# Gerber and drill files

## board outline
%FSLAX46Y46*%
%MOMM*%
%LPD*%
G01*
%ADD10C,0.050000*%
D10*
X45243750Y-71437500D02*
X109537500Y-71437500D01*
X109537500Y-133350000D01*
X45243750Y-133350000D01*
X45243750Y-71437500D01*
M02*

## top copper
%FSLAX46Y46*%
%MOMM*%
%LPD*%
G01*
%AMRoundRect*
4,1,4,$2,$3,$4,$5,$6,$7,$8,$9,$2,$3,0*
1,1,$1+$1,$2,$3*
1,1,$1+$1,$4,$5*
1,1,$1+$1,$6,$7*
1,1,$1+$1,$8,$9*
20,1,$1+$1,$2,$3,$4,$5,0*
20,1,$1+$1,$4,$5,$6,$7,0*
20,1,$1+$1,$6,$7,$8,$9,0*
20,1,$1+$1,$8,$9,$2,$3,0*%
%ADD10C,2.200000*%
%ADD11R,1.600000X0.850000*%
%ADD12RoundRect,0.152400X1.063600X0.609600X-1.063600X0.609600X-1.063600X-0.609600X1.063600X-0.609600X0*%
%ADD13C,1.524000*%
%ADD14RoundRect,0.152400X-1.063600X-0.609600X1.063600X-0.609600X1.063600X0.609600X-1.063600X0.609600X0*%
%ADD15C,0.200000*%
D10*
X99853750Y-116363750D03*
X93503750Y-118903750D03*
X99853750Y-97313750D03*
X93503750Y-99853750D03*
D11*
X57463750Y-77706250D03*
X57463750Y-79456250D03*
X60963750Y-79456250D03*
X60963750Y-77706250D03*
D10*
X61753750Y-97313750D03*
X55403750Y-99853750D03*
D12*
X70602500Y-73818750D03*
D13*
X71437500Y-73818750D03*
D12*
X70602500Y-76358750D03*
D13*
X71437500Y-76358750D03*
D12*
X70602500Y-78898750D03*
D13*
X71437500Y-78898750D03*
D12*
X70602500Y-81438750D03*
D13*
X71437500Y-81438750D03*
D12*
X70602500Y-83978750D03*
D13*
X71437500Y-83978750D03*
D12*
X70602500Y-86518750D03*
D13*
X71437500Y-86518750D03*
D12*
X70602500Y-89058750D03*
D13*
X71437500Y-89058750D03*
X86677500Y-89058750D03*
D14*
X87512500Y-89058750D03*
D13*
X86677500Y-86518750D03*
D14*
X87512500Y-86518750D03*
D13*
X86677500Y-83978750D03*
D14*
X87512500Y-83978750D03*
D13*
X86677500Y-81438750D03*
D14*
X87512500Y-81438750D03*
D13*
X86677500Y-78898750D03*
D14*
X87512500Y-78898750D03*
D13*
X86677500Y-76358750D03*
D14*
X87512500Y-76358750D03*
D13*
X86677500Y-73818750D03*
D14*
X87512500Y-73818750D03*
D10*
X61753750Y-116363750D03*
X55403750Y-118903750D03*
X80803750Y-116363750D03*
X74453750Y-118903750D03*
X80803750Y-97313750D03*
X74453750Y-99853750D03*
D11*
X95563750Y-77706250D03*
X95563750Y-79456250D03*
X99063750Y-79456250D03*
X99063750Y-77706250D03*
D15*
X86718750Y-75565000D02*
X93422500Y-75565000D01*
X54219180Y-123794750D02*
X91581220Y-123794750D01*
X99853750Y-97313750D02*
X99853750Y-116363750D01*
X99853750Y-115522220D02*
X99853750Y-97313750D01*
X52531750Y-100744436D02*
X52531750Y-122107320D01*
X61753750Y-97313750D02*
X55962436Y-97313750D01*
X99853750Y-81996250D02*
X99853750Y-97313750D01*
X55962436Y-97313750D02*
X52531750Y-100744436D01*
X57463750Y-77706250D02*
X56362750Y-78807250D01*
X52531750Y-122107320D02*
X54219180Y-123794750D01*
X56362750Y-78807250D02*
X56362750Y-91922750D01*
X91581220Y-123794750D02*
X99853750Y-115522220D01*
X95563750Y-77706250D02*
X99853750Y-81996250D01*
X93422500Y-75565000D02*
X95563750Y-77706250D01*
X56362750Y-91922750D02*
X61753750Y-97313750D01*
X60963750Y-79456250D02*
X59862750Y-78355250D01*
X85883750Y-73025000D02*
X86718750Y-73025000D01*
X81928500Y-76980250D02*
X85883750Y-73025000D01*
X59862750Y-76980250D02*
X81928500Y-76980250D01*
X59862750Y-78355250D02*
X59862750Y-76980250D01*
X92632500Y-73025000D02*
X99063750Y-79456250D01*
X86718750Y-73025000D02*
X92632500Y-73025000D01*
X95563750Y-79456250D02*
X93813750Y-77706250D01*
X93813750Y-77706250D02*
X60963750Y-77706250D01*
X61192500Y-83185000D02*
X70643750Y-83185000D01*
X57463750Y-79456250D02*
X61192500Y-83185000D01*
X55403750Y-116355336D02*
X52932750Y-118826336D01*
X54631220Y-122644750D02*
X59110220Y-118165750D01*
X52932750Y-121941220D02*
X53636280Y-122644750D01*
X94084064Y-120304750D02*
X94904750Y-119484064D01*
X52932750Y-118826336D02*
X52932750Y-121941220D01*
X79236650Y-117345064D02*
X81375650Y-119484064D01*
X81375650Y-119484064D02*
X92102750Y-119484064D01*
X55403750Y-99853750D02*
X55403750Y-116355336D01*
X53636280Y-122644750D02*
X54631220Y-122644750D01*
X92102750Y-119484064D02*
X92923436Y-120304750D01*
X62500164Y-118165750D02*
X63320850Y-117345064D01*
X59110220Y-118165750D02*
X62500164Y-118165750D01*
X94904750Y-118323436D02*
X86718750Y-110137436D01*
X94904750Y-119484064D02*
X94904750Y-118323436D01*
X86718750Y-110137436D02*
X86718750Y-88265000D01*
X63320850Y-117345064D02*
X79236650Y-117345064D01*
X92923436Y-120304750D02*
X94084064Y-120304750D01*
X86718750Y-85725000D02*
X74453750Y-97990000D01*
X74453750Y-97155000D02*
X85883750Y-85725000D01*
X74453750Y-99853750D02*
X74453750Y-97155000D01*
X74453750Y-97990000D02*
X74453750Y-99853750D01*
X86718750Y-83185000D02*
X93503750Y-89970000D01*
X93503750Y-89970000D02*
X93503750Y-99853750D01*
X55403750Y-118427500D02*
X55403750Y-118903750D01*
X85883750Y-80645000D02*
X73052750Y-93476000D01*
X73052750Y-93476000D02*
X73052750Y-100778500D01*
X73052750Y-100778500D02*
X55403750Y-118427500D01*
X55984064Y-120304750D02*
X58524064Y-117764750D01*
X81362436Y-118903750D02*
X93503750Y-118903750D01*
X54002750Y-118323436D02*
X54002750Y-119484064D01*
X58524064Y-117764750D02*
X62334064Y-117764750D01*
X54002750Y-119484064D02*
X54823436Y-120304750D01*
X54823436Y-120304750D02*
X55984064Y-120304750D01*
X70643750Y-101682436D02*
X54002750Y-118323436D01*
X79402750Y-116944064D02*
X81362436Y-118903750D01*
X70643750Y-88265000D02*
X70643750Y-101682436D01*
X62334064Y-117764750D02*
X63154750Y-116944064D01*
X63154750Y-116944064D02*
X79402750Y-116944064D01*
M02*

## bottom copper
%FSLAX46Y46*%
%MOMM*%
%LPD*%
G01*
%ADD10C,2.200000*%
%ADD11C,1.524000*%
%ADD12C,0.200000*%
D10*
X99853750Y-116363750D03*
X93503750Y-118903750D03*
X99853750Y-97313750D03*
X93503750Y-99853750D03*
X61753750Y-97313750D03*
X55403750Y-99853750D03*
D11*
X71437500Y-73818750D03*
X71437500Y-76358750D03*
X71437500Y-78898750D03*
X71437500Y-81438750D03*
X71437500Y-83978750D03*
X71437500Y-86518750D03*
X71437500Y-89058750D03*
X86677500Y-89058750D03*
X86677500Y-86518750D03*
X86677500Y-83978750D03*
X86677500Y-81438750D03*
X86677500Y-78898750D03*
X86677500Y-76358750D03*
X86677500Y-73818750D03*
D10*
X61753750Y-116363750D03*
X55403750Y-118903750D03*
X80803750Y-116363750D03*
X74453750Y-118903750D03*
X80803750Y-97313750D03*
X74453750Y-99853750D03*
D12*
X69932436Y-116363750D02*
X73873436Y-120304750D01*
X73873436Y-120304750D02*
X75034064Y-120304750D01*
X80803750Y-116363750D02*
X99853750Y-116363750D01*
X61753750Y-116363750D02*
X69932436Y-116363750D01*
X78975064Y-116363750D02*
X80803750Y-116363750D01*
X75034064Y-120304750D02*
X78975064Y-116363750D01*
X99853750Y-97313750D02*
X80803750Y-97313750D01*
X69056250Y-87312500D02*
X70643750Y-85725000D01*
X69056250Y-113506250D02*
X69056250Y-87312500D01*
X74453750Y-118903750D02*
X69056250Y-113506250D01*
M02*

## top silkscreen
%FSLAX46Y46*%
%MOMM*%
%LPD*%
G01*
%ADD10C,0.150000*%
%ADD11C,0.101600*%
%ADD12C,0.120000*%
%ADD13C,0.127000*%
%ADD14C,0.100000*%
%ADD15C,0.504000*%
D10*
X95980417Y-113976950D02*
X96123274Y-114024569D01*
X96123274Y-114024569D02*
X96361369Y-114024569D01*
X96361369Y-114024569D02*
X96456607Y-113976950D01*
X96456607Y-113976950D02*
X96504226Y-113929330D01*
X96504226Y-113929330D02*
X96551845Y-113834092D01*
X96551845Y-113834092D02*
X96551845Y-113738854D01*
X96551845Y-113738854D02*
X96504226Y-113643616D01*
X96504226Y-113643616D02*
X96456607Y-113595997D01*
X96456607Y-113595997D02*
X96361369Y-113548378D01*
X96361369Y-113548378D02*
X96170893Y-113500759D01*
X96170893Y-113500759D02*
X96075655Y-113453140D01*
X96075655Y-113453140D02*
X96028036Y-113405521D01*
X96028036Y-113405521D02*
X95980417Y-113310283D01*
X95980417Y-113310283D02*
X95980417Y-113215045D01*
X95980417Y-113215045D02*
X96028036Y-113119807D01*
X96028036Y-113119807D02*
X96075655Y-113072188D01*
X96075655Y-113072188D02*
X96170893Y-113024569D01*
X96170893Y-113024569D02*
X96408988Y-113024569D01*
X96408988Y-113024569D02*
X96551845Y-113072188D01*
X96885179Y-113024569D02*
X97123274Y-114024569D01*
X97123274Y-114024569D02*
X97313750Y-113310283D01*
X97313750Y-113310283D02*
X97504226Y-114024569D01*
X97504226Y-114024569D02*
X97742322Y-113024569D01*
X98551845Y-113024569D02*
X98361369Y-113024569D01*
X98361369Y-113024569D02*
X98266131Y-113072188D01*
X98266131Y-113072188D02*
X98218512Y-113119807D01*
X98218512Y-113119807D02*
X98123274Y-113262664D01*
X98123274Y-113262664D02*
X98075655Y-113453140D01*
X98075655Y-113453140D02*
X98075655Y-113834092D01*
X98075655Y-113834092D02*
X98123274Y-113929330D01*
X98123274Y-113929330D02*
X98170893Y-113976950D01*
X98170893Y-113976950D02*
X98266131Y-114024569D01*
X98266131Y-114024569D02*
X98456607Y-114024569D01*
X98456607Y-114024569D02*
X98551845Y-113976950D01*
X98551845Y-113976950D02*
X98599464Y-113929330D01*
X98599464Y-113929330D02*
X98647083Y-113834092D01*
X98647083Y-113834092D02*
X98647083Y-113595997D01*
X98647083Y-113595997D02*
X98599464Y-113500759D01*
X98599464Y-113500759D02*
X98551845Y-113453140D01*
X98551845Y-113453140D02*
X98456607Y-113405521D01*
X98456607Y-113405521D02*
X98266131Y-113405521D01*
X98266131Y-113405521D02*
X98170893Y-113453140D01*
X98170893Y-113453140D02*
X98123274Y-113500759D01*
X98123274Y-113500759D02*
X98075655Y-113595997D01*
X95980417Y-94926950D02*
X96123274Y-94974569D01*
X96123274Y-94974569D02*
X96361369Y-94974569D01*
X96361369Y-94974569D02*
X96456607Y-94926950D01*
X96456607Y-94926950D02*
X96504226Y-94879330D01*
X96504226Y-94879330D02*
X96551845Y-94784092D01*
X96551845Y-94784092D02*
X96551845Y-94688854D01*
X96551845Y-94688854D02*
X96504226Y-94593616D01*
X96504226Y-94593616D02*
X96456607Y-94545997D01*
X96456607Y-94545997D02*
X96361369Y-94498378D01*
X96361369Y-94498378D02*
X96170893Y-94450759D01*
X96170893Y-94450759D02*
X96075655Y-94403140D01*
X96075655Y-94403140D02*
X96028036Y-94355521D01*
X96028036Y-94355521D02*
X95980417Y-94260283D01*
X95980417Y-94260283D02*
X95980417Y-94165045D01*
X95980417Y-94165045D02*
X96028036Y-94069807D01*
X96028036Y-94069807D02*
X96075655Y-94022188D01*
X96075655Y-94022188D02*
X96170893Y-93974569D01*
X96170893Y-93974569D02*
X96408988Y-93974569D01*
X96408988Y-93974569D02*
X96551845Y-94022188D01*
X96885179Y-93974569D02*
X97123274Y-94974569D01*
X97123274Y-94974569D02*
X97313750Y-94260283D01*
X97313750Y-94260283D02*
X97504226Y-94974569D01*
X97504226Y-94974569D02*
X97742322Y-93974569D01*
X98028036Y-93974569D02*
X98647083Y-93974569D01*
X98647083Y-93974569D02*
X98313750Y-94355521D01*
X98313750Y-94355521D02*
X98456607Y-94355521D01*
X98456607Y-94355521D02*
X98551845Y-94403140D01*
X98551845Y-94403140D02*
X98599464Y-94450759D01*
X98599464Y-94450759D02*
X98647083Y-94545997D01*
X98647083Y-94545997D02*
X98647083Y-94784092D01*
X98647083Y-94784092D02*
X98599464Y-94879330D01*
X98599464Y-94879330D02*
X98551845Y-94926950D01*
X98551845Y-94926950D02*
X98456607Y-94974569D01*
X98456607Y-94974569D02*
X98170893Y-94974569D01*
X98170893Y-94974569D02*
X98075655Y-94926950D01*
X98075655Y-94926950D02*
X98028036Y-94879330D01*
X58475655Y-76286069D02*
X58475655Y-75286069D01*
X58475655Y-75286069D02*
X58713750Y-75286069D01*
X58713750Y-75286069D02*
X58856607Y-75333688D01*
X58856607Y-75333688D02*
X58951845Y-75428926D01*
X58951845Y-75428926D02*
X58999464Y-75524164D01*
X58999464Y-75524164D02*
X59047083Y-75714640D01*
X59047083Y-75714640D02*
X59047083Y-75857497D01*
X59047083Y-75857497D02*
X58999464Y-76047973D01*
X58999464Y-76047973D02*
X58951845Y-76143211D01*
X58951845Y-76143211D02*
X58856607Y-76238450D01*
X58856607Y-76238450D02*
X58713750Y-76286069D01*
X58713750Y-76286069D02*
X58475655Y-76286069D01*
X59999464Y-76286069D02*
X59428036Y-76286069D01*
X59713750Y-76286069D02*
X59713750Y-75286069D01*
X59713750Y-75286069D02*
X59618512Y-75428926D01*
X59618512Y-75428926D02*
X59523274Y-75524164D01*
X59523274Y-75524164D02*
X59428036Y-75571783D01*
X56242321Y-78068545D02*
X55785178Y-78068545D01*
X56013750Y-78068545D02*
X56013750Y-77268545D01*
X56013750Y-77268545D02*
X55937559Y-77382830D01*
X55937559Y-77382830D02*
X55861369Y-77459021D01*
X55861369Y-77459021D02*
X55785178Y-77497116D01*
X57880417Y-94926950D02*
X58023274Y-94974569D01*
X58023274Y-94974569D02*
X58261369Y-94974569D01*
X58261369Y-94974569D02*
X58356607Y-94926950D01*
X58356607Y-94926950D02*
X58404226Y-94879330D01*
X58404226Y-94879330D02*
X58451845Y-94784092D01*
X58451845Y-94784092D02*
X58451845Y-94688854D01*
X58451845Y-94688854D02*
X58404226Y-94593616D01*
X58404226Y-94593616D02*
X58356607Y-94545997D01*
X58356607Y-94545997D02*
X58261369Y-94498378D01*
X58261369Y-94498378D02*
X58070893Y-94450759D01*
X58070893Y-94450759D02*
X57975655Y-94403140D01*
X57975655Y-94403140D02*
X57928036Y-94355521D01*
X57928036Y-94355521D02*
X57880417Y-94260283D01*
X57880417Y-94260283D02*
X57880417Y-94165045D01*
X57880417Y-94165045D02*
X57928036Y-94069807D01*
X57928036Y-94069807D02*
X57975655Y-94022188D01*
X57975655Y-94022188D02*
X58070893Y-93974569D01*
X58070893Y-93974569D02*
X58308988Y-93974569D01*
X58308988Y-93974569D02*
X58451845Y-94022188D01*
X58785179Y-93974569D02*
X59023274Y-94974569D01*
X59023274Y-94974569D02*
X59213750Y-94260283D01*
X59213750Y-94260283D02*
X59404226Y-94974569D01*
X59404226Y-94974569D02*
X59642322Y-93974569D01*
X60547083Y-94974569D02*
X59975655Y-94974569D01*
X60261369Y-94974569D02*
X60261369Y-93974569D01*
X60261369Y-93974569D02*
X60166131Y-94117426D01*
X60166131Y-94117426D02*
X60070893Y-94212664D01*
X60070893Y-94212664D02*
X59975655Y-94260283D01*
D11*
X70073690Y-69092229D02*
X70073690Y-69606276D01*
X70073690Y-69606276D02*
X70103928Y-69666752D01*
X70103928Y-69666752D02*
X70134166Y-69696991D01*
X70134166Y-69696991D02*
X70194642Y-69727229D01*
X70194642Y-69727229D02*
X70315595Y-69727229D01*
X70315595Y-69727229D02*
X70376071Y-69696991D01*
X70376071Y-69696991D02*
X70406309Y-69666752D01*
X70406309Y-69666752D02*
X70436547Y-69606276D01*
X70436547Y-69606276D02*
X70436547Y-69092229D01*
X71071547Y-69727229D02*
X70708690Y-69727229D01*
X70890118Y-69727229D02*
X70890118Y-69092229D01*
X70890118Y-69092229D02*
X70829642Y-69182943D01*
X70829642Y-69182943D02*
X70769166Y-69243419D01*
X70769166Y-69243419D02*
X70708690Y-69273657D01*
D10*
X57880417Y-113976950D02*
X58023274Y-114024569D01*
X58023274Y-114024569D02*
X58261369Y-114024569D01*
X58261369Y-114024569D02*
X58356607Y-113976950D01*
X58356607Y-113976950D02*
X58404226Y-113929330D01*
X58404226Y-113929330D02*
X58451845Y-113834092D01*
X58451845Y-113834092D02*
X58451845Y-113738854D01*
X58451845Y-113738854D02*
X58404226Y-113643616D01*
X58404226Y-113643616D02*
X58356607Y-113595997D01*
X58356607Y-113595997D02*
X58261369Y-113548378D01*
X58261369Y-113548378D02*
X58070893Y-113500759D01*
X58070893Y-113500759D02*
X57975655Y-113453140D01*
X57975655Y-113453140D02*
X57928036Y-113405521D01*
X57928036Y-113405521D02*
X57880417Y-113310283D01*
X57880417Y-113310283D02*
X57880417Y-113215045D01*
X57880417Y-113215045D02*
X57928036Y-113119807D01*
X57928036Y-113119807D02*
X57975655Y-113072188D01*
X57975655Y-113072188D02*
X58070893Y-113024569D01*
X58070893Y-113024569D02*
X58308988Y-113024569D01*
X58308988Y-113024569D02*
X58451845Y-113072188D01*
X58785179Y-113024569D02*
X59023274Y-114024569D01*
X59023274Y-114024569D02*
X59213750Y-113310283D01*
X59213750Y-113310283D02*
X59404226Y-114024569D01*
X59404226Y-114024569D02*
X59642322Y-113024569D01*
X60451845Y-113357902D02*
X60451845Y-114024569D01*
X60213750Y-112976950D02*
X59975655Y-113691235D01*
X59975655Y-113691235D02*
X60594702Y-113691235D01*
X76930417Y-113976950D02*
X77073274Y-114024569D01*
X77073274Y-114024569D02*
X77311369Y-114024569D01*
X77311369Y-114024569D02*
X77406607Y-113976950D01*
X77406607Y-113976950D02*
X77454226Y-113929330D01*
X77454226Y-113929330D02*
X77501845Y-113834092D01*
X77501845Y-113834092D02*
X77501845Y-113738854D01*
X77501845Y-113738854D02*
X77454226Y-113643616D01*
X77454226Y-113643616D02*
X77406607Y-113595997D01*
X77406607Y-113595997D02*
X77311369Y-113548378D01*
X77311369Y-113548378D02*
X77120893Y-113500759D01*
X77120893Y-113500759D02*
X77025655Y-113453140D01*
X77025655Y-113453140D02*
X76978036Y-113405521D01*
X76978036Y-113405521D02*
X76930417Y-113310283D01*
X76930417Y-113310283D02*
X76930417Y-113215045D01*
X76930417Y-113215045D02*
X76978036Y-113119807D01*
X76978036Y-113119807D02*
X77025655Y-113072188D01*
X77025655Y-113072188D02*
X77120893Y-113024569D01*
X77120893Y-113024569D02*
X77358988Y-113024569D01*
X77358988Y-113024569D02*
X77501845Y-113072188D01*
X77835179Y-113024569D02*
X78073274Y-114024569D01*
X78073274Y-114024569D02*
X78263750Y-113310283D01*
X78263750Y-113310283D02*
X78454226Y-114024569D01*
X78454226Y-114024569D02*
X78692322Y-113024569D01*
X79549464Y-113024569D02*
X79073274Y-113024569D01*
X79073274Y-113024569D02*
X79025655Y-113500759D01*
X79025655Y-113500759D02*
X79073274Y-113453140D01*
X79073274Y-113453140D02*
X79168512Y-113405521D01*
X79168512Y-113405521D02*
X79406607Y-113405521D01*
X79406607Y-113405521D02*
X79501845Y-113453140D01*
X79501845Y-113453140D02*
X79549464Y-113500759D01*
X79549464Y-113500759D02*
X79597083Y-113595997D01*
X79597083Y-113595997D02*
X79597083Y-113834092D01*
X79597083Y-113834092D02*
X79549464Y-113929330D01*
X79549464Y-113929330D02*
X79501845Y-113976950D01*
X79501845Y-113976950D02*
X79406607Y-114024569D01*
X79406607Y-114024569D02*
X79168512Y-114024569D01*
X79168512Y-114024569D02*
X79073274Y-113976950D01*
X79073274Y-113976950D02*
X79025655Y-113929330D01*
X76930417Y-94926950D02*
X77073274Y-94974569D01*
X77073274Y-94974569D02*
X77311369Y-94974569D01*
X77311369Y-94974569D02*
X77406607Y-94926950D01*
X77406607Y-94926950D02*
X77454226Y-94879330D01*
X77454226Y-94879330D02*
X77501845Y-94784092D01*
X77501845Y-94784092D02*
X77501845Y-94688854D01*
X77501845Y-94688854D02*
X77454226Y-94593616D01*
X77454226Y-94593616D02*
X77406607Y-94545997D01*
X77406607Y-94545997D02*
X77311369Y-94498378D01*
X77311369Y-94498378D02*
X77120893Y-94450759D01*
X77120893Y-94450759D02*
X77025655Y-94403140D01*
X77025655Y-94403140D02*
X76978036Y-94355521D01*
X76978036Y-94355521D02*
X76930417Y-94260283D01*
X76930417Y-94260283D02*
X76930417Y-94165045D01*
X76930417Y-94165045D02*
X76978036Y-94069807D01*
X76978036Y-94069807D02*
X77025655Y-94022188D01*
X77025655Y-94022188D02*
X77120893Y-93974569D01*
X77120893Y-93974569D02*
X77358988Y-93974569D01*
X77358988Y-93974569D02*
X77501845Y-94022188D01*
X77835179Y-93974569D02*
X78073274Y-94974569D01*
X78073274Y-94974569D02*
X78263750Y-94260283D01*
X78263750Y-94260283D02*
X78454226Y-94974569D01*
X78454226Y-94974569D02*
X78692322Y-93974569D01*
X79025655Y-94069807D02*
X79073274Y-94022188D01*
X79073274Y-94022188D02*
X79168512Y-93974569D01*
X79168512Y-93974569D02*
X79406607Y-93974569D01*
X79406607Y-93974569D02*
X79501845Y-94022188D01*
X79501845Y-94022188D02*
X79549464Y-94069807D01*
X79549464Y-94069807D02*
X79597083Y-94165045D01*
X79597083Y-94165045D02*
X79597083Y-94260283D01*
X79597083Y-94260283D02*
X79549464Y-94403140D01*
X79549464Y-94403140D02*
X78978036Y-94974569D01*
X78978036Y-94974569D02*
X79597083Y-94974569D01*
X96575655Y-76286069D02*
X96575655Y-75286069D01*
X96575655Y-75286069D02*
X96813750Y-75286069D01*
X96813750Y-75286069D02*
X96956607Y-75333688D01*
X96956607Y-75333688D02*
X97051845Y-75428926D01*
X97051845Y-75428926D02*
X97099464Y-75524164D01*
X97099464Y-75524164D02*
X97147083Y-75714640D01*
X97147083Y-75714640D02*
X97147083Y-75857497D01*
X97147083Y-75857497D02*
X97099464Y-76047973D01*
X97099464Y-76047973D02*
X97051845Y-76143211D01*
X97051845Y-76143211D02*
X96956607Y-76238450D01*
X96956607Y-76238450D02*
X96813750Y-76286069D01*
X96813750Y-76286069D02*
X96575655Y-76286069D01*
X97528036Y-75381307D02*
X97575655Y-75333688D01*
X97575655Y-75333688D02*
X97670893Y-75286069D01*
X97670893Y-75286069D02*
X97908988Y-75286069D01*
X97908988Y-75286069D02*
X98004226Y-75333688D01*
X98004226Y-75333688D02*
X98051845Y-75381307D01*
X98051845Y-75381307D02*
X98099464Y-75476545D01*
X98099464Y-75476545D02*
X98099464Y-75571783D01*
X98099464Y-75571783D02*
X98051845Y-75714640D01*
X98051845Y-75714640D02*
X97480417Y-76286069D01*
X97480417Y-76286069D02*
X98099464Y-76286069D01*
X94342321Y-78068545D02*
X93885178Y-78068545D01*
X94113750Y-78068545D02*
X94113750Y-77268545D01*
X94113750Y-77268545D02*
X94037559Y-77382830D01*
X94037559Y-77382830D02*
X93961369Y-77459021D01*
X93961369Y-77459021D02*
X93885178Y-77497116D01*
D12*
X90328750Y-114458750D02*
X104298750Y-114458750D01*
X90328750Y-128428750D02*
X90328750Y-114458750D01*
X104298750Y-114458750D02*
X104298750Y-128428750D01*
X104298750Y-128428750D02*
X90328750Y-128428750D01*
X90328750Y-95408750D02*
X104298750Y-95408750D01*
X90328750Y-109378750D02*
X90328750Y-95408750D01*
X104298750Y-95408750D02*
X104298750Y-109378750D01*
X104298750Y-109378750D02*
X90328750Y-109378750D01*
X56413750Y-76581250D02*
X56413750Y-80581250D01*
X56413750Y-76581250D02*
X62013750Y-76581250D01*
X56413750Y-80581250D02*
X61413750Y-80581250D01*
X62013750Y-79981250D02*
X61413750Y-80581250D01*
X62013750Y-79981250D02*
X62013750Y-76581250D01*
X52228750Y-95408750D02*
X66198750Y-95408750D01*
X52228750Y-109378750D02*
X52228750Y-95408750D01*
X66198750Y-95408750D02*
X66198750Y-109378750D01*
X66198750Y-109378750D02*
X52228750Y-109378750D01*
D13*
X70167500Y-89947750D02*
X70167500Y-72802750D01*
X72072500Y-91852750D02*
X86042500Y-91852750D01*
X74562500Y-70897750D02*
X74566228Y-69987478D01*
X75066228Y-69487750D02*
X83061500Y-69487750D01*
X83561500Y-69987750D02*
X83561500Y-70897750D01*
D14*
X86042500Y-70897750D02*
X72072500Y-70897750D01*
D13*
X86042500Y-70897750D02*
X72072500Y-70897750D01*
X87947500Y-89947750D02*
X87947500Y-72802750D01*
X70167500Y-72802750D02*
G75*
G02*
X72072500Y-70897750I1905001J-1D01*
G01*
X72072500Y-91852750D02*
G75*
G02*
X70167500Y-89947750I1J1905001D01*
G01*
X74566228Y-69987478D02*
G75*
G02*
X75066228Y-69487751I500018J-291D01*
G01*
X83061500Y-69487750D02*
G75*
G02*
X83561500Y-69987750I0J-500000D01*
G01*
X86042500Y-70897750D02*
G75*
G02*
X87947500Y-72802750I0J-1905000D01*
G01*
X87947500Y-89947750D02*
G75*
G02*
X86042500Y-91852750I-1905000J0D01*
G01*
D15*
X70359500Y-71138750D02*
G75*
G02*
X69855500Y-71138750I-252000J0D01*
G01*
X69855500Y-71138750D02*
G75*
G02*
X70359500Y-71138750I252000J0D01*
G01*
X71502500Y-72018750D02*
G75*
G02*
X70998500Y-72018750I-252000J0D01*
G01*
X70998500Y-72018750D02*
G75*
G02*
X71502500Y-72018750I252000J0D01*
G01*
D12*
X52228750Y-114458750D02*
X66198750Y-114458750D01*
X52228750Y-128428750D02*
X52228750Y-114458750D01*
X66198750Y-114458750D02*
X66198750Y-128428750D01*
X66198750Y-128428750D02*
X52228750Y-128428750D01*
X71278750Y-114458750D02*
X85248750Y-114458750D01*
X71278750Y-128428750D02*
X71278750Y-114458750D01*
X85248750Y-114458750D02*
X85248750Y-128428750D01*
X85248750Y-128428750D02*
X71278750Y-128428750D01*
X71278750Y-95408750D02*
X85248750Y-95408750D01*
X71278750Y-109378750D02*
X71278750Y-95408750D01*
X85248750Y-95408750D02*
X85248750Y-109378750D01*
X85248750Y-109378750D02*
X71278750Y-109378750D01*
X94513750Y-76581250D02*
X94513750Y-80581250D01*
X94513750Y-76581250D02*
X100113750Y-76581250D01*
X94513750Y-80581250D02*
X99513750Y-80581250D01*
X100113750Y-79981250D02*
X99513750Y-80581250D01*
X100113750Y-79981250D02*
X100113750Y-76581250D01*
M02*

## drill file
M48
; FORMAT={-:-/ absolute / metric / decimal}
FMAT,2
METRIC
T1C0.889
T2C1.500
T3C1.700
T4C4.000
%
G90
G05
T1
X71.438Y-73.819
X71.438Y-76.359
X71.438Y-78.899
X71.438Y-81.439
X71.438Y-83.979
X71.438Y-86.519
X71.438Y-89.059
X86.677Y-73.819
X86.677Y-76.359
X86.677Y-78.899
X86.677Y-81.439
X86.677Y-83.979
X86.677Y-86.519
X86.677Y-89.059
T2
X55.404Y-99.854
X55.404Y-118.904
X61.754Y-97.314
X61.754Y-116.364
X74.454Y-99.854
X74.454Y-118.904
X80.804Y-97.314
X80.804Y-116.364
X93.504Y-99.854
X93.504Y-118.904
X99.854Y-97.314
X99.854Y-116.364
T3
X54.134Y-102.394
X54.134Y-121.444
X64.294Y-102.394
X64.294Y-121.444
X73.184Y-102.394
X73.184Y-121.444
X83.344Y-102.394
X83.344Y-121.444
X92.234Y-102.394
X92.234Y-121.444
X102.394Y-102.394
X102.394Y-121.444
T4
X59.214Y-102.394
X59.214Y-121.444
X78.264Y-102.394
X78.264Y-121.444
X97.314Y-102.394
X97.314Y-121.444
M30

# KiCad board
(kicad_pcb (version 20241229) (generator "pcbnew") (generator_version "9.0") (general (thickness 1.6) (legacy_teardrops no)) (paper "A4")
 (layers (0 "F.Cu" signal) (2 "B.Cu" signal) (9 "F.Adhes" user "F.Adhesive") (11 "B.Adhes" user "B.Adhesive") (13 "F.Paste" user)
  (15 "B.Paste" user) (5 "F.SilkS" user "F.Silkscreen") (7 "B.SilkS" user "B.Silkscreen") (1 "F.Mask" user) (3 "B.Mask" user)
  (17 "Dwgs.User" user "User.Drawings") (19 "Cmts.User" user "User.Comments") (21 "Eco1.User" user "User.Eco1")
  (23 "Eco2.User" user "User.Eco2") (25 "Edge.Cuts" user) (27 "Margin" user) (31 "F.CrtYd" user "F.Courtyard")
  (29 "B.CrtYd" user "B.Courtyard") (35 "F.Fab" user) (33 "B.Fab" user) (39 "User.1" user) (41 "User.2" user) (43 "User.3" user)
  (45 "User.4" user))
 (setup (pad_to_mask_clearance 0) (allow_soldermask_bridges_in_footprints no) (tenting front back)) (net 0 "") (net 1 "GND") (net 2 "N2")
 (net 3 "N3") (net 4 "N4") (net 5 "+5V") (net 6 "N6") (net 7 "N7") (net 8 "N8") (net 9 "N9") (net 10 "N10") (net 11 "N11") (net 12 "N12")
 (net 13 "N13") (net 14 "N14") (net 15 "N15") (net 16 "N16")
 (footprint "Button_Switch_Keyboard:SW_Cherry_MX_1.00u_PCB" (layer "F.Cu") (at 99.85375 116.36375)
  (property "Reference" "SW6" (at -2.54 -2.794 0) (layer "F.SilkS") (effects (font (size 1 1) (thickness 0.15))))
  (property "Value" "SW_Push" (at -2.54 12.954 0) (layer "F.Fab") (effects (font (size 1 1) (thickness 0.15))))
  (fp_line (start -9.525 -1.905) (end 4.445 -1.905) (stroke (width 0.12) (type solid)) (layer "F.SilkS"))
  (fp_line (start -9.525 12.065) (end -9.525 -1.905) (stroke (width 0.12) (type solid)) (layer "F.SilkS"))
  (fp_line (start 4.445 -1.905) (end 4.445 12.065) (stroke (width 0.12) (type solid)) (layer "F.SilkS"))
  (fp_line (start 4.445 12.065) (end -9.525 12.065) (stroke (width 0.12) (type solid)) (layer "F.SilkS"))
  (pad "" np_thru_hole circle (at -7.62 5.08) (size 1.7 1.7) (drill 1.7) (layers "*.Cu" "*.Mask"))
  (pad "" np_thru_hole circle (at -2.54 5.08) (size 4 4) (drill 4) (layers "*.Cu" "*.Mask"))
  (pad "" np_thru_hole circle (at 2.54 5.08) (size 1.7 1.7) (drill 1.7) (layers "*.Cu" "*.Mask"))
  (pad "1" thru_hole circle (at 0 0) (size 2.2 2.2) (drill 1.5) (layers "*.Cu" "*.Mask") (remove_unused_layers no) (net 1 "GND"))
  (pad "2" thru_hole circle (at -6.35 2.54) (size 2.2 2.2) (drill 1.5) (layers "*.Cu" "*.Mask") (remove_unused_layers no) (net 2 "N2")))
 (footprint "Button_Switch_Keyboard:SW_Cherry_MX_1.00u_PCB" (layer "F.Cu") (at 99.85375 97.31375)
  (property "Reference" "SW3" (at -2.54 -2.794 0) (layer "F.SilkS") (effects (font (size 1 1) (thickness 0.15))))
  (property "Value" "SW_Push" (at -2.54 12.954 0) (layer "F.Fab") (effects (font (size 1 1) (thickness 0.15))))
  (fp_line (start -9.525 -1.905) (end 4.445 -1.905) (stroke (width 0.12) (type solid)) (layer "F.SilkS"))
  (fp_line (start -9.525 12.065) (end -9.525 -1.905) (stroke (width 0.12) (type solid)) (layer "F.SilkS"))
  (fp_line (start 4.445 -1.905) (end 4.445 12.065) (stroke (width 0.12) (type solid)) (layer "F.SilkS"))
  (fp_line (start 4.445 12.065) (end -9.525 12.065) (stroke (width 0.12) (type solid)) (layer "F.SilkS"))
  (pad "" np_thru_hole circle (at -7.62 5.08) (size 1.7 1.7) (drill 1.7) (layers "*.Cu" "*.Mask"))
  (pad "" np_thru_hole circle (at -2.54 5.08) (size 4 4) (drill 4) (layers "*.Cu" "*.Mask"))
  (pad "" np_thru_hole circle (at 2.54 5.08) (size 1.7 1.7) (drill 1.7) (layers "*.Cu" "*.Mask"))
  (pad "1" thru_hole circle (at 0 0) (size 2.2 2.2) (drill 1.5) (layers "*.Cu" "*.Mask") (remove_unused_layers no) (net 1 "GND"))
  (pad "2" thru_hole circle (at -6.35 2.54) (size 2.2 2.2) (drill 1.5) (layers "*.Cu" "*.Mask") (remove_unused_layers no) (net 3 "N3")))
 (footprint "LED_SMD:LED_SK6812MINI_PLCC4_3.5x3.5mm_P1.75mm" (layer "F.Cu") (at 59.21375 78.58125)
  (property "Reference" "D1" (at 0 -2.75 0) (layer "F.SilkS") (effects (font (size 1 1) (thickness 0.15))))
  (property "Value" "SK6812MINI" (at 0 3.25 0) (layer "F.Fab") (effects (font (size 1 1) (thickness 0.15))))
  (fp_line (start -2.8 -2) (end -2.8 2) (stroke (width 0.12) (type default)) (layer "F.SilkS"))
  (fp_line (start -2.8 -2) (end 2.8 -2) (stroke (width 0.12) (type solid)) (layer "F.SilkS"))
  (fp_line (start -2.8 2) (end 2.2 2) (stroke (width 0.12) (type solid)) (layer "F.SilkS"))
  (fp_line (start 2.8 1.4) (end 2.2 2) (stroke (width 0.12) (type default)) (layer "F.SilkS"))
  (fp_line (start 2.8 1.4) (end 2.8 -2) (stroke (width 0.12) (type solid)) (layer "F.SilkS"))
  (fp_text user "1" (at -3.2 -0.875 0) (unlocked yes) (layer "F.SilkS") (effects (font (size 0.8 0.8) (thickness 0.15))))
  (pad "1" smd rect (at -1.75 -0.875) (size 1.6 0.85) (layers "F.Cu" "F.Mask" "F.Paste") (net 1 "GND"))
  (pad "2" smd rect (at -1.75 0.875) (size 1.6 0.85) (layers "F.Cu" "F.Mask" "F.Paste") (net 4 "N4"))
  (pad "3" smd rect (at 1.75 0.875) (size 1.6 0.85) (layers "F.Cu" "F.Mask" "F.Paste") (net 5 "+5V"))
  (pad "4" smd rect (at 1.75 -0.875) (size 1.6 0.85) (layers "F.Cu" "F.Mask" "F.Paste") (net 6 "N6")))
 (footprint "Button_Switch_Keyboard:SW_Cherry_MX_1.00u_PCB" (layer "F.Cu") (at 61.75375 97.31375)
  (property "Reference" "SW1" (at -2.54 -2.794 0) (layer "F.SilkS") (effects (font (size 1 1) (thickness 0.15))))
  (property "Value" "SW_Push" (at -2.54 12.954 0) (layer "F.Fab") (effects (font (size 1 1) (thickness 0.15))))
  (fp_line (start -9.525 -1.905) (end 4.445 -1.905) (stroke (width 0.12) (type solid)) (layer "F.SilkS"))
  (fp_line (start -9.525 12.065) (end -9.525 -1.905) (stroke (width 0.12) (type solid)) (layer "F.SilkS"))
  (fp_line (start 4.445 -1.905) (end 4.445 12.065) (stroke (width 0.12) (type solid)) (layer "F.SilkS"))
  (fp_line (start 4.445 12.065) (end -9.525 12.065) (stroke (width 0.12) (type solid)) (layer "F.SilkS"))
  (pad "" np_thru_hole circle (at -7.62 5.08) (size 1.7 1.7) (drill 1.7) (layers "*.Cu" "*.Mask"))
  (pad "" np_thru_hole circle (at -2.54 5.08) (size 4 4) (drill 4) (layers "*.Cu" "*.Mask"))
  (pad "" np_thru_hole circle (at 2.54 5.08) (size 1.7 1.7) (drill 1.7) (layers "*.Cu" "*.Mask"))
  (pad "1" thru_hole circle (at 0 0) (size 2.2 2.2) (drill 1.5) (layers "*.Cu" "*.Mask") (remove_unused_layers no) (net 1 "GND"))
  (pad "2" thru_hole circle (at -6.35 2.54) (size 2.2 2.2) (drill 1.5) (layers "*.Cu" "*.Mask") (remove_unused_layers no) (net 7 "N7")))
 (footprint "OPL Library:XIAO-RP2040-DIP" (layer "F.Cu") (at 79.0575 81.43875)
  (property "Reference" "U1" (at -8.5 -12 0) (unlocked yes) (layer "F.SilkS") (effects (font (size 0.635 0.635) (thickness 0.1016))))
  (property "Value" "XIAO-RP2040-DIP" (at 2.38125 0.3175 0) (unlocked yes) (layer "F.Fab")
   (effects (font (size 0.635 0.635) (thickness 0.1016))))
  (fp_line (start -8.89 8.509) (end -8.89 -8.636) (stroke (width 0.127) (type solid)) (layer "F.SilkS"))
  (fp_line (start -6.985 10.414) (end 6.985 10.414) (stroke (width 0.127) (type solid)) (layer "F.SilkS"))
  (fp_line (start -4.495 -10.541) (end -4.491272 -11.451272) (stroke (width 0.127) (type solid)) (layer "F.SilkS"))
  (fp_line (start -3.991272 -11.951) (end 4.004 -11.951) (stroke (width 0.127) (type solid)) (layer "F.SilkS"))
  (fp_line (start 4.504 -11.451) (end 4.504 -10.541) (stroke (width 0.127) (type solid)) (layer "F.SilkS"))
  (fp_line (start 6.985 -10.541) (end -6.985 -10.541) (stroke (width 0.1) (type solid)) (layer "F.SilkS"))
  (fp_line (start 6.985 -10.541) (end -6.985 -10.541) (stroke (width 0.127) (type solid)) (layer "F.SilkS"))
  (fp_line (start 8.89 8.509) (end 8.89 -8.636) (stroke (width 0.127) (type solid)) (layer "F.SilkS"))
  (fp_arc (start -8.89 -8.636) (mid -8.332038 -9.983038) (end -6.985 -10.541) (stroke (width 0.127) (type solid)) (layer "F.SilkS"))
  (fp_arc (start -6.985 10.414) (mid -8.332038 9.856038) (end -8.89 8.509) (stroke (width 0.127) (type solid)) (layer "F.SilkS"))
  (fp_arc (start -4.491272 -11.451272) (mid -4.344728 -11.80464) (end -3.991272 -11.951) (stroke (width 0.127) (type default))
   (layer "F.SilkS"))
  (fp_arc (start 4.004 -11.951) (mid 4.357553 -11.804553) (end 4.504 -11.451) (stroke (width 0.127) (type default)) (layer "F.SilkS"))
  (fp_arc (start 6.985 -10.541) (mid 8.332038 -9.983038) (end 8.89 -8.636) (stroke (width 0.127) (type solid)) (layer "F.SilkS"))
  (fp_arc (start 8.89 8.509) (mid 8.332038 9.856038) (end 6.985 10.414) (stroke (width 0.127) (type solid)) (layer "F.SilkS"))
  (fp_circle (center -8.95 -10.3) (end -8.95 -10.554) (stroke (width 0.5) (type solid)) (fill yes) (layer "F.SilkS"))
  (fp_circle (center -7.807 -9.42) (end -7.807 -9.674) (stroke (width 0.5) (type solid)) (fill yes) (layer "F.SilkS"))
  (pad "1" smd roundrect (at -8.455 -7.62 180) (size 2.432 1.524) (layers "F.Cu" "F.Mask") (roundrect_rratio 0.1) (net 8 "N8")
   (thermal_bridge_angle 45))
  (pad "1" thru_hole circle (at -7.62 -7.62 180) (size 1.524 1.524) (drill 0.889) (layers "*.Cu" "*.Mask") (remove_unused_layers no)
   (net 8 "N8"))
  (pad "2" smd roundrect (at -8.455 -5.08 180) (size 2.432 1.524) (layers "F.Cu" "F.Mask") (roundrect_rratio 0.1) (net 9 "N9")
   (thermal_bridge_angle 45))
  (pad "2" thru_hole circle (at -7.62 -5.08 180) (size 1.524 1.524) (drill 0.889) (layers "*.Cu" "*.Mask") (remove_unused_layers no)
   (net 9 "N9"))
  (pad "3" smd roundrect (at -8.455 -2.54 180) (size 2.432 1.524) (layers "F.Cu" "F.Mask") (roundrect_rratio 0.1) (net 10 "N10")
   (thermal_bridge_angle 45))
  (pad "3" thru_hole circle (at -7.62 -2.54 180) (size 1.524 1.524) (drill 0.889) (layers "*.Cu" "*.Mask") (remove_unused_layers no)
   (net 10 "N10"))
  (pad "4" smd roundrect (at -8.455 0 180) (size 2.432 1.524) (layers "F.Cu" "F.Mask") (roundrect_rratio 0.1) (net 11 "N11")
   (thermal_bridge_angle 45))
  (pad "4" thru_hole circle (at -7.62 0 180) (size 1.524 1.524) (drill 0.889) (layers "*.Cu" "*.Mask") (remove_unused_layers no)
   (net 11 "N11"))
  (pad "5" smd roundrect (at -8.455 2.54 180) (size 2.432 1.524) (layers "F.Cu" "F.Mask") (roundrect_rratio 0.1) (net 4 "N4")
   (thermal_bridge_angle 45))
  (pad "5" thru_hole circle (at -7.62 2.54 180) (size 1.524 1.524) (drill 0.889) (layers "*.Cu" "*.Mask") (remove_unused_layers no)
   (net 4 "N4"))
  (pad "6" smd roundrect (at -8.455 5.08 180) (size 2.432 1.524) (layers "F.Cu" "F.Mask") (roundrect_rratio 0.1) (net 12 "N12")
   (thermal_bridge_angle 45))
  (pad "6" thru_hole circle (at -7.62 5.08 180) (size 1.524 1.524) (drill 0.889) (layers "*.Cu" "*.Mask") (remove_unused_layers no)
   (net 12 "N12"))
  (pad "7" smd roundrect (at -8.455 7.62 180) (size 2.432 1.524) (layers "F.Cu" "F.Mask") (roundrect_rratio 0.1) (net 2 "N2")
   (thermal_bridge_angle 45))
  (pad "7" thru_hole circle (at -7.62 7.62 180) (size 1.524 1.524) (drill 0.889) (layers "*.Cu" "*.Mask") (remove_unused_layers no)
   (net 2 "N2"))
  (pad "8" thru_hole circle (at 7.62 7.62) (size 1.524 1.524) (drill 0.889) (layers "*.Cu" "*.Mask") (remove_unused_layers no) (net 7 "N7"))
  (pad "8" smd roundrect (at 8.455 7.62) (size 2.432 1.524) (layers "F.Cu" "F.Mask") (roundrect_rratio 0.1) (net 7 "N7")
   (thermal_bridge_angle 45))
  (pad "9" thru_hole circle (at 7.62 5.08) (size 1.524 1.524) (drill 0.889) (layers "*.Cu" "*.Mask") (remove_unused_layers no)
   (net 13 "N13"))
  (pad "9" smd roundrect (at 8.455 5.08) (size 2.432 1.524) (layers "F.Cu" "F.Mask") (roundrect_rratio 0.1) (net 13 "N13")
   (thermal_bridge_angle 45))
  (pad "10" thru_hole circle (at 7.62 2.54) (size 1.524 1.524) (drill 0.889) (layers "*.Cu" "*.Mask") (remove_unused_layers no) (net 3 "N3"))
  (pad "10" smd roundrect (at 8.455 2.54) (size 2.432 1.524) (layers "F.Cu" "F.Mask") (roundrect_rratio 0.1) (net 3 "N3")
   (thermal_bridge_angle 45))
  (pad "11" thru_hole circle (at 7.62 0) (size 1.524 1.524) (drill 0.889) (layers "*.Cu" "*.Mask") (remove_unused_layers no) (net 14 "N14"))
  (pad "11" smd roundrect (at 8.455 0) (size 2.432 1.524) (layers "F.Cu" "F.Mask") (roundrect_rratio 0.1) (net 14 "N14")
   (thermal_bridge_angle 45))
  (pad "12" thru_hole circle (at 7.62 -2.54) (size 1.524 1.524) (drill 0.889) (layers "*.Cu" "*.Mask") (remove_unused_layers no)
   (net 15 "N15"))
  (pad "12" smd roundrect (at 8.455 -2.54) (size 2.432 1.524) (layers "F.Cu" "F.Mask") (roundrect_rratio 0.1) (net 15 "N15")
   (thermal_bridge_angle 45))
  (pad "13" thru_hole circle (at 7.62 -5.08) (size 1.524 1.524) (drill 0.889) (layers "*.Cu" "*.Mask") (remove_unused_layers no)
   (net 1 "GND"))
  (pad "13" smd roundrect (at 8.455 -5.08) (size 2.432 1.524) (layers "F.Cu" "F.Mask") (roundrect_rratio 0.1) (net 1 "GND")
   (thermal_bridge_angle 45))
  (pad "14" thru_hole circle (at 7.62 -7.62) (size 1.524 1.524) (drill 0.889) (layers "*.Cu" "*.Mask") (remove_unused_layers no)
   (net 5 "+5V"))
  (pad "14" smd roundrect (at 8.455 -7.62) (size 2.432 1.524) (layers "F.Cu" "F.Mask") (roundrect_rratio 0.1) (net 5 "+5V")
   (thermal_bridge_angle 45)))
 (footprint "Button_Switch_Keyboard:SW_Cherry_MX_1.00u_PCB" (layer "F.Cu") (at 61.75375 116.36375)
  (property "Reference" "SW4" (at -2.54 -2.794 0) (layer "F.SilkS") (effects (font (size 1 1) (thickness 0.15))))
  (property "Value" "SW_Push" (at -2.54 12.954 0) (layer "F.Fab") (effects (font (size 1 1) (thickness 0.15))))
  (fp_line (start -9.525 -1.905) (end 4.445 -1.905) (stroke (width 0.12) (type solid)) (layer "F.SilkS"))
  (fp_line (start -9.525 12.065) (end -9.525 -1.905) (stroke (width 0.12) (type solid)) (layer "F.SilkS"))
  (fp_line (start 4.445 -1.905) (end 4.445 12.065) (stroke (width 0.12) (type solid)) (layer "F.SilkS"))
  (fp_line (start 4.445 12.065) (end -9.525 12.065) (stroke (width 0.12) (type solid)) (layer "F.SilkS"))
  (pad "" np_thru_hole circle (at -7.62 5.08) (size 1.7 1.7) (drill 1.7) (layers "*.Cu" "*.Mask"))
  (pad "" np_thru_hole circle (at -2.54 5.08) (size 4 4) (drill 4) (layers "*.Cu" "*.Mask"))
  (pad "" np_thru_hole circle (at 2.54 5.08) (size 1.7 1.7) (drill 1.7) (layers "*.Cu" "*.Mask"))
  (pad "1" thru_hole circle (at 0 0) (size 2.2 2.2) (drill 1.5) (layers "*.Cu" "*.Mask") (remove_unused_layers no) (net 1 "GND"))
  (pad "2" thru_hole circle (at -6.35 2.54) (size 2.2 2.2) (drill 1.5) (layers "*.Cu" "*.Mask") (remove_unused_layers no) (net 14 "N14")))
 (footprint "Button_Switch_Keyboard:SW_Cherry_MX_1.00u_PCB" (layer "F.Cu") (at 80.80375 116.36375)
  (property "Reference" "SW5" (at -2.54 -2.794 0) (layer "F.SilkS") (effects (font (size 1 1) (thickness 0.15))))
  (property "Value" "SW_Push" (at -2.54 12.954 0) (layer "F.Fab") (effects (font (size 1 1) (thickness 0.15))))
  (fp_line (start -9.525 -1.905) (end 4.445 -1.905) (stroke (width 0.12) (type solid)) (layer "F.SilkS"))
  (fp_line (start -9.525 12.065) (end -9.525 -1.905) (stroke (width 0.12) (type solid)) (layer "F.SilkS"))
  (fp_line (start 4.445 -1.905) (end 4.445 12.065) (stroke (width 0.12) (type solid)) (layer "F.SilkS"))
  (fp_line (start 4.445 12.065) (end -9.525 12.065) (stroke (width 0.12) (type solid)) (layer "F.SilkS"))
  (pad "" np_thru_hole circle (at -7.62 5.08) (size 1.7 1.7) (drill 1.7) (layers "*.Cu" "*.Mask"))
  (pad "" np_thru_hole circle (at -2.54 5.08) (size 4 4) (drill 4) (layers "*.Cu" "*.Mask"))
  (pad "" np_thru_hole circle (at 2.54 5.08) (size 1.7 1.7) (drill 1.7) (layers "*.Cu" "*.Mask"))
  (pad "1" thru_hole circle (at 0 0) (size 2.2 2.2) (drill 1.5) (layers "*.Cu" "*.Mask") (remove_unused_layers no) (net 1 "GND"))
  (pad "2" thru_hole circle (at -6.35 2.54) (size 2.2 2.2) (drill 1.5) (layers "*.Cu" "*.Mask") (remove_unused_layers no) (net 12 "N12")))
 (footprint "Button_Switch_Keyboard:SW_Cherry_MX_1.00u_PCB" (layer "F.Cu") (at 80.80375 97.31375)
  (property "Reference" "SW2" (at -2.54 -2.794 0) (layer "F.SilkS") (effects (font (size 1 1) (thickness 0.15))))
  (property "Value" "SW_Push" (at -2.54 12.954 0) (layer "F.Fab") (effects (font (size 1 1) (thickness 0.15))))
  (fp_line (start -9.525 -1.905) (end 4.445 -1.905) (stroke (width 0.12) (type solid)) (layer "F.SilkS"))
  (fp_line (start -9.525 12.065) (end -9.525 -1.905) (stroke (width 0.12) (type solid)) (layer "F.SilkS"))
  (fp_line (start 4.445 -1.905) (end 4.445 12.065) (stroke (width 0.12) (type solid)) (layer "F.SilkS"))
  (fp_line (start 4.445 12.065) (end -9.525 12.065) (stroke (width 0.12) (type solid)) (layer "F.SilkS"))
  (pad "" np_thru_hole circle (at -7.62 5.08) (size 1.7 1.7) (drill 1.7) (layers "*.Cu" "*.Mask"))
  (pad "" np_thru_hole circle (at -2.54 5.08) (size 4 4) (drill 4) (layers "*.Cu" "*.Mask"))
  (pad "" np_thru_hole circle (at 2.54 5.08) (size 1.7 1.7) (drill 1.7) (layers "*.Cu" "*.Mask"))
  (pad "1" thru_hole circle (at 0 0) (size 2.2 2.2) (drill 1.5) (layers "*.Cu" "*.Mask") (remove_unused_layers no) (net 1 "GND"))
  (pad "2" thru_hole circle (at -6.35 2.54) (size 2.2 2.2) (drill 1.5) (layers "*.Cu" "*.Mask") (remove_unused_layers no) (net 13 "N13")))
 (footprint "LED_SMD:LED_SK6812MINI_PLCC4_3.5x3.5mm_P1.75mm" (layer "F.Cu") (at 97.31375 78.58125)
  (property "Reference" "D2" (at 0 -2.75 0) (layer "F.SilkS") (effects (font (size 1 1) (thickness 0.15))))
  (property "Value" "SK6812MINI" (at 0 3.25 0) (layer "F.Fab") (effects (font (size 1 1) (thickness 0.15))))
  (fp_line (start -2.8 -2) (end -2.8 2) (stroke (width 0.12) (type default)) (layer "F.SilkS"))
  (fp_line (start -2.8 -2) (end 2.8 -2) (stroke (width 0.12) (type solid)) (layer "F.SilkS"))
  (fp_line (start -2.8 2) (end 2.2 2) (stroke (width 0.12) (type solid)) (layer "F.SilkS"))
  (fp_line (start 2.8 1.4) (end 2.2 2) (stroke (width 0.12) (type default)) (layer "F.SilkS"))
  (fp_line (start 2.8 1.4) (end 2.8 -2) (stroke (width 0.12) (type solid)) (layer "F.SilkS"))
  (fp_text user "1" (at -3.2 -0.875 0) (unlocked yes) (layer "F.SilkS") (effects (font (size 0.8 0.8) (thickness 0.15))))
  (pad "1" smd rect (at -1.75 -0.875) (size 1.6 0.85) (layers "F.Cu" "F.Mask" "F.Paste") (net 1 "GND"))
  (pad "2" smd rect (at -1.75 0.875) (size 1.6 0.85) (layers "F.Cu" "F.Mask" "F.Paste") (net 6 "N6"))
  (pad "3" smd rect (at 1.75 0.875) (size 1.6 0.85) (layers "F.Cu" "F.Mask" "F.Paste") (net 5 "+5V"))
  (pad "4" smd rect (at 1.75 -0.875) (size 1.6 0.85) (layers "F.Cu" "F.Mask" "F.Paste") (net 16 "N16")))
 (gr_rect (start 45.24375 71.4375) (end 109.5375 133.35) (stroke (width 0.05) (type default)) (fill no) (layer "Edge.Cuts"))
 (segment (start 86.71875 75.565) (end 93.4225 75.565) (width 0.2) (layer "F.Cu") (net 1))
 (segment (start 54.21918 123.79475) (end 91.58122 123.79475) (width 0.2) (layer "F.Cu") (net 1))
 (segment (start 99.85375 97.31375) (end 99.85375 116.36375) (width 0.2) (layer "F.Cu") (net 1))
 (segment (start 99.85375 115.52222) (end 99.85375 97.31375) (width 0.2) (layer "F.Cu") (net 1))
 (segment (start 52.53175 100.744436) (end 52.53175 122.10732) (width 0.2) (layer "F.Cu") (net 1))
 (segment (start 61.75375 97.31375) (end 55.962436 97.31375) (width 0.2) (layer "F.Cu") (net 1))
 (segment (start 99.85375 81.99625) (end 99.85375 97.31375) (width 0.2) (layer "F.Cu") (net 1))
 (segment (start 55.962436 97.31375) (end 52.53175 100.744436) (width 0.2) (layer "F.Cu") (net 1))
 (segment (start 57.46375 77.70625) (end 56.36275 78.80725) (width 0.2) (layer "F.Cu") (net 1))
 (segment (start 52.53175 122.10732) (end 54.21918 123.79475) (width 0.2) (layer "F.Cu") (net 1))
 (segment (start 56.36275 78.80725) (end 56.36275 91.92275) (width 0.2) (layer "F.Cu") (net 1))
 (segment (start 91.58122 123.79475) (end 99.85375 115.52222) (width 0.2) (layer "F.Cu") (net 1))
 (segment (start 95.56375 77.70625) (end 99.85375 81.99625) (width 0.2) (layer "F.Cu") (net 1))
 (segment (start 93.4225 75.565) (end 95.56375 77.70625) (width 0.2) (layer "F.Cu") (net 1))
 (segment (start 56.36275 91.92275) (end 61.75375 97.31375) (width 0.2) (layer "F.Cu") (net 1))
 (segment (start 69.932436 116.36375) (end 73.873436 120.30475) (width 0.2) (layer "B.Cu") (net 1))
 (segment (start 73.873436 120.30475) (end 75.034064 120.30475) (width 0.2) (layer "B.Cu") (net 1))
 (segment (start 80.80375 116.36375) (end 99.85375 116.36375) (width 0.2) (layer "B.Cu") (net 1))
 (segment (start 61.75375 116.36375) (end 69.932436 116.36375) (width 0.2) (layer "B.Cu") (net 1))
 (segment (start 78.975064 116.36375) (end 80.80375 116.36375) (width 0.2) (layer "B.Cu") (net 1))
 (segment (start 75.034064 120.30475) (end 78.975064 116.36375) (width 0.2) (layer "B.Cu") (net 1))
 (segment (start 99.85375 97.31375) (end 80.80375 97.31375) (width 0.2) (layer "B.Cu") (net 1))
 (segment (start 60.96375 79.45625) (end 59.86275 78.35525) (width 0.2) (layer "F.Cu") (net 5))
 (segment (start 85.88375 73.025) (end 86.71875 73.025) (width 0.2) (layer "F.Cu") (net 5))
 (segment (start 81.9285 76.98025) (end 85.88375 73.025) (width 0.2) (layer "F.Cu") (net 5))
 (segment (start 59.86275 76.98025) (end 81.9285 76.98025) (width 0.2) (layer "F.Cu") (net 5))
 (segment (start 59.86275 78.35525) (end 59.86275 76.98025) (width 0.2) (layer "F.Cu") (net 5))
 (segment (start 92.6325 73.025) (end 99.06375 79.45625) (width 0.2) (layer "F.Cu") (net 5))
 (segment (start 86.71875 73.025) (end 92.6325 73.025) (width 0.2) (layer "F.Cu") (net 5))
 (segment (start 95.56375 79.45625) (end 93.81375 77.70625) (width 0.2) (layer "F.Cu") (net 6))
 (segment (start 93.81375 77.70625) (end 60.96375 77.70625) (width 0.2) (layer "F.Cu") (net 6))
 (segment (start 61.1925 83.185) (end 70.64375 83.185) (width 0.2) (layer "F.Cu") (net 4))
 (segment (start 57.46375 79.45625) (end 61.1925 83.185) (width 0.2) (layer "F.Cu") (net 4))
 (segment (start 55.40375 116.355336) (end 52.93275 118.826336) (width 0.2) (layer "F.Cu") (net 7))
 (segment (start 54.63122 122.64475) (end 59.11022 118.16575) (width 0.2) (layer "F.Cu") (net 7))
 (segment (start 52.93275 121.94122) (end 53.63628 122.64475) (width 0.2) (layer "F.Cu") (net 7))
 (segment (start 94.084064 120.30475) (end 94.90475 119.484064) (width 0.2) (layer "F.Cu") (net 7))
 (segment (start 52.93275 118.826336) (end 52.93275 121.94122) (width 0.2) (layer "F.Cu") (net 7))
 (segment (start 79.23665 117.345064) (end 81.37565 119.484064) (width 0.2) (layer "F.Cu") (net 7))
 (segment (start 81.37565 119.484064) (end 92.10275 119.484064) (width 0.2) (layer "F.Cu") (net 7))
 (segment (start 55.40375 99.85375) (end 55.40375 116.355336) (width 0.2) (layer "F.Cu") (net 7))
 (segment (start 53.63628 122.64475) (end 54.63122 122.64475) (width 0.2) (layer "F.Cu") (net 7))
 (segment (start 92.10275 119.484064) (end 92.923436 120.30475) (width 0.2) (layer "F.Cu") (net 7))
 (segment (start 62.500164 118.16575) (end 63.32085 117.345064) (width 0.2) (layer "F.Cu") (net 7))
 (segment (start 59.11022 118.16575) (end 62.500164 118.16575) (width 0.2) (layer "F.Cu") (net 7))
 (segment (start 94.90475 118.323436) (end 86.71875 110.137436) (width 0.2) (layer "F.Cu") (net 7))
 (segment (start 94.90475 119.484064) (end 94.90475 118.323436) (width 0.2) (layer "F.Cu") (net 7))
 (segment (start 86.71875 110.137436) (end 86.71875 88.265) (width 0.2) (layer "F.Cu") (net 7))
 (segment (start 63.32085 117.345064) (end 79.23665 117.345064) (width 0.2) (layer "F.Cu") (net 7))
 (segment (start 92.923436 120.30475) (end 94.084064 120.30475) (width 0.2) (layer "F.Cu") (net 7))
 (segment (start 86.71875 85.725) (end 74.45375 97.99) (width 0.2) (layer "F.Cu") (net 13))
 (segment (start 74.45375 97.155) (end 85.88375 85.725) (width 0.2) (layer "F.Cu") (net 13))
 (segment (start 74.45375 99.85375) (end 74.45375 97.155) (width 0.2) (layer "F.Cu") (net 13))
 (segment (start 74.45375 97.99) (end 74.45375 99.85375) (width 0.2) (layer "F.Cu") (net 13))
 (segment (start 86.71875 83.185) (end 93.50375 89.97) (width 0.2) (layer "F.Cu") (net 3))
 (segment (start 93.50375 89.97) (end 93.50375 99.85375) (width 0.2) (layer "F.Cu") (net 3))
 (segment (start 55.40375 118.4275) (end 55.40375 118.90375) (width 0.2) (layer "F.Cu") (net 14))
 (segment (start 85.88375 80.645) (end 73.05275 93.476) (width 0.2) (layer "F.Cu") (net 14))
 (segment (start 73.05275 93.476) (end 73.05275 100.7785) (width 0.2) (layer "F.Cu") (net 14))
 (segment (start 73.05275 100.7785) (end 55.40375 118.4275) (width 0.2) (layer "F.Cu") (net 14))
 (segment (start 69.05625 87.3125) (end 70.64375 85.725) (width 0.2) (layer "B.Cu") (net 12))
 (segment (start 69.05625 113.50625) (end 69.05625 87.3125) (width 0.2) (layer "B.Cu") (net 12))
 (segment (start 74.45375 118.90375) (end 69.05625 113.50625) (width 0.2) (layer "B.Cu") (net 12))
 (segment (start 55.984064 120.30475) (end 58.524064 117.76475) (width 0.2) (layer "F.Cu") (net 2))
 (segment (start 81.362436 118.90375) (end 93.50375 118.90375) (width 0.2) (layer "F.Cu") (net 2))
 (segment (start 54.00275 118.323436) (end 54.00275 119.484064) (width 0.2) (layer "F.Cu") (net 2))
 (segment (start 58.524064 117.76475) (end 62.334064 117.76475) (width 0.2) (layer "F.Cu") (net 2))
 (segment (start 54.00275 119.484064) (end 54.823436 120.30475) (width 0.2) (layer "F.Cu") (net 2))
 (segment (start 54.823436 120.30475) (end 55.984064 120.30475) (width 0.2) (layer "F.Cu") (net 2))
 (segment (start 70.64375 101.682436) (end 54.00275 118.323436) (width 0.2) (layer "F.Cu") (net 2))
 (segment (start 79.40275 116.944064) (end 81.362436 118.90375) (width 0.2) (layer "F.Cu") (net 2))
 (segment (start 70.64375 88.265) (end 70.64375 101.682436) (width 0.2) (layer "F.Cu") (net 2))
 (segment (start 62.334064 117.76475) (end 63.15475 116.944064) (width 0.2) (layer "F.Cu") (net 2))
 (segment (start 63.15475 116.944064) (end 79.40275 116.944064) (width 0.2) (layer "F.Cu") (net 2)))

